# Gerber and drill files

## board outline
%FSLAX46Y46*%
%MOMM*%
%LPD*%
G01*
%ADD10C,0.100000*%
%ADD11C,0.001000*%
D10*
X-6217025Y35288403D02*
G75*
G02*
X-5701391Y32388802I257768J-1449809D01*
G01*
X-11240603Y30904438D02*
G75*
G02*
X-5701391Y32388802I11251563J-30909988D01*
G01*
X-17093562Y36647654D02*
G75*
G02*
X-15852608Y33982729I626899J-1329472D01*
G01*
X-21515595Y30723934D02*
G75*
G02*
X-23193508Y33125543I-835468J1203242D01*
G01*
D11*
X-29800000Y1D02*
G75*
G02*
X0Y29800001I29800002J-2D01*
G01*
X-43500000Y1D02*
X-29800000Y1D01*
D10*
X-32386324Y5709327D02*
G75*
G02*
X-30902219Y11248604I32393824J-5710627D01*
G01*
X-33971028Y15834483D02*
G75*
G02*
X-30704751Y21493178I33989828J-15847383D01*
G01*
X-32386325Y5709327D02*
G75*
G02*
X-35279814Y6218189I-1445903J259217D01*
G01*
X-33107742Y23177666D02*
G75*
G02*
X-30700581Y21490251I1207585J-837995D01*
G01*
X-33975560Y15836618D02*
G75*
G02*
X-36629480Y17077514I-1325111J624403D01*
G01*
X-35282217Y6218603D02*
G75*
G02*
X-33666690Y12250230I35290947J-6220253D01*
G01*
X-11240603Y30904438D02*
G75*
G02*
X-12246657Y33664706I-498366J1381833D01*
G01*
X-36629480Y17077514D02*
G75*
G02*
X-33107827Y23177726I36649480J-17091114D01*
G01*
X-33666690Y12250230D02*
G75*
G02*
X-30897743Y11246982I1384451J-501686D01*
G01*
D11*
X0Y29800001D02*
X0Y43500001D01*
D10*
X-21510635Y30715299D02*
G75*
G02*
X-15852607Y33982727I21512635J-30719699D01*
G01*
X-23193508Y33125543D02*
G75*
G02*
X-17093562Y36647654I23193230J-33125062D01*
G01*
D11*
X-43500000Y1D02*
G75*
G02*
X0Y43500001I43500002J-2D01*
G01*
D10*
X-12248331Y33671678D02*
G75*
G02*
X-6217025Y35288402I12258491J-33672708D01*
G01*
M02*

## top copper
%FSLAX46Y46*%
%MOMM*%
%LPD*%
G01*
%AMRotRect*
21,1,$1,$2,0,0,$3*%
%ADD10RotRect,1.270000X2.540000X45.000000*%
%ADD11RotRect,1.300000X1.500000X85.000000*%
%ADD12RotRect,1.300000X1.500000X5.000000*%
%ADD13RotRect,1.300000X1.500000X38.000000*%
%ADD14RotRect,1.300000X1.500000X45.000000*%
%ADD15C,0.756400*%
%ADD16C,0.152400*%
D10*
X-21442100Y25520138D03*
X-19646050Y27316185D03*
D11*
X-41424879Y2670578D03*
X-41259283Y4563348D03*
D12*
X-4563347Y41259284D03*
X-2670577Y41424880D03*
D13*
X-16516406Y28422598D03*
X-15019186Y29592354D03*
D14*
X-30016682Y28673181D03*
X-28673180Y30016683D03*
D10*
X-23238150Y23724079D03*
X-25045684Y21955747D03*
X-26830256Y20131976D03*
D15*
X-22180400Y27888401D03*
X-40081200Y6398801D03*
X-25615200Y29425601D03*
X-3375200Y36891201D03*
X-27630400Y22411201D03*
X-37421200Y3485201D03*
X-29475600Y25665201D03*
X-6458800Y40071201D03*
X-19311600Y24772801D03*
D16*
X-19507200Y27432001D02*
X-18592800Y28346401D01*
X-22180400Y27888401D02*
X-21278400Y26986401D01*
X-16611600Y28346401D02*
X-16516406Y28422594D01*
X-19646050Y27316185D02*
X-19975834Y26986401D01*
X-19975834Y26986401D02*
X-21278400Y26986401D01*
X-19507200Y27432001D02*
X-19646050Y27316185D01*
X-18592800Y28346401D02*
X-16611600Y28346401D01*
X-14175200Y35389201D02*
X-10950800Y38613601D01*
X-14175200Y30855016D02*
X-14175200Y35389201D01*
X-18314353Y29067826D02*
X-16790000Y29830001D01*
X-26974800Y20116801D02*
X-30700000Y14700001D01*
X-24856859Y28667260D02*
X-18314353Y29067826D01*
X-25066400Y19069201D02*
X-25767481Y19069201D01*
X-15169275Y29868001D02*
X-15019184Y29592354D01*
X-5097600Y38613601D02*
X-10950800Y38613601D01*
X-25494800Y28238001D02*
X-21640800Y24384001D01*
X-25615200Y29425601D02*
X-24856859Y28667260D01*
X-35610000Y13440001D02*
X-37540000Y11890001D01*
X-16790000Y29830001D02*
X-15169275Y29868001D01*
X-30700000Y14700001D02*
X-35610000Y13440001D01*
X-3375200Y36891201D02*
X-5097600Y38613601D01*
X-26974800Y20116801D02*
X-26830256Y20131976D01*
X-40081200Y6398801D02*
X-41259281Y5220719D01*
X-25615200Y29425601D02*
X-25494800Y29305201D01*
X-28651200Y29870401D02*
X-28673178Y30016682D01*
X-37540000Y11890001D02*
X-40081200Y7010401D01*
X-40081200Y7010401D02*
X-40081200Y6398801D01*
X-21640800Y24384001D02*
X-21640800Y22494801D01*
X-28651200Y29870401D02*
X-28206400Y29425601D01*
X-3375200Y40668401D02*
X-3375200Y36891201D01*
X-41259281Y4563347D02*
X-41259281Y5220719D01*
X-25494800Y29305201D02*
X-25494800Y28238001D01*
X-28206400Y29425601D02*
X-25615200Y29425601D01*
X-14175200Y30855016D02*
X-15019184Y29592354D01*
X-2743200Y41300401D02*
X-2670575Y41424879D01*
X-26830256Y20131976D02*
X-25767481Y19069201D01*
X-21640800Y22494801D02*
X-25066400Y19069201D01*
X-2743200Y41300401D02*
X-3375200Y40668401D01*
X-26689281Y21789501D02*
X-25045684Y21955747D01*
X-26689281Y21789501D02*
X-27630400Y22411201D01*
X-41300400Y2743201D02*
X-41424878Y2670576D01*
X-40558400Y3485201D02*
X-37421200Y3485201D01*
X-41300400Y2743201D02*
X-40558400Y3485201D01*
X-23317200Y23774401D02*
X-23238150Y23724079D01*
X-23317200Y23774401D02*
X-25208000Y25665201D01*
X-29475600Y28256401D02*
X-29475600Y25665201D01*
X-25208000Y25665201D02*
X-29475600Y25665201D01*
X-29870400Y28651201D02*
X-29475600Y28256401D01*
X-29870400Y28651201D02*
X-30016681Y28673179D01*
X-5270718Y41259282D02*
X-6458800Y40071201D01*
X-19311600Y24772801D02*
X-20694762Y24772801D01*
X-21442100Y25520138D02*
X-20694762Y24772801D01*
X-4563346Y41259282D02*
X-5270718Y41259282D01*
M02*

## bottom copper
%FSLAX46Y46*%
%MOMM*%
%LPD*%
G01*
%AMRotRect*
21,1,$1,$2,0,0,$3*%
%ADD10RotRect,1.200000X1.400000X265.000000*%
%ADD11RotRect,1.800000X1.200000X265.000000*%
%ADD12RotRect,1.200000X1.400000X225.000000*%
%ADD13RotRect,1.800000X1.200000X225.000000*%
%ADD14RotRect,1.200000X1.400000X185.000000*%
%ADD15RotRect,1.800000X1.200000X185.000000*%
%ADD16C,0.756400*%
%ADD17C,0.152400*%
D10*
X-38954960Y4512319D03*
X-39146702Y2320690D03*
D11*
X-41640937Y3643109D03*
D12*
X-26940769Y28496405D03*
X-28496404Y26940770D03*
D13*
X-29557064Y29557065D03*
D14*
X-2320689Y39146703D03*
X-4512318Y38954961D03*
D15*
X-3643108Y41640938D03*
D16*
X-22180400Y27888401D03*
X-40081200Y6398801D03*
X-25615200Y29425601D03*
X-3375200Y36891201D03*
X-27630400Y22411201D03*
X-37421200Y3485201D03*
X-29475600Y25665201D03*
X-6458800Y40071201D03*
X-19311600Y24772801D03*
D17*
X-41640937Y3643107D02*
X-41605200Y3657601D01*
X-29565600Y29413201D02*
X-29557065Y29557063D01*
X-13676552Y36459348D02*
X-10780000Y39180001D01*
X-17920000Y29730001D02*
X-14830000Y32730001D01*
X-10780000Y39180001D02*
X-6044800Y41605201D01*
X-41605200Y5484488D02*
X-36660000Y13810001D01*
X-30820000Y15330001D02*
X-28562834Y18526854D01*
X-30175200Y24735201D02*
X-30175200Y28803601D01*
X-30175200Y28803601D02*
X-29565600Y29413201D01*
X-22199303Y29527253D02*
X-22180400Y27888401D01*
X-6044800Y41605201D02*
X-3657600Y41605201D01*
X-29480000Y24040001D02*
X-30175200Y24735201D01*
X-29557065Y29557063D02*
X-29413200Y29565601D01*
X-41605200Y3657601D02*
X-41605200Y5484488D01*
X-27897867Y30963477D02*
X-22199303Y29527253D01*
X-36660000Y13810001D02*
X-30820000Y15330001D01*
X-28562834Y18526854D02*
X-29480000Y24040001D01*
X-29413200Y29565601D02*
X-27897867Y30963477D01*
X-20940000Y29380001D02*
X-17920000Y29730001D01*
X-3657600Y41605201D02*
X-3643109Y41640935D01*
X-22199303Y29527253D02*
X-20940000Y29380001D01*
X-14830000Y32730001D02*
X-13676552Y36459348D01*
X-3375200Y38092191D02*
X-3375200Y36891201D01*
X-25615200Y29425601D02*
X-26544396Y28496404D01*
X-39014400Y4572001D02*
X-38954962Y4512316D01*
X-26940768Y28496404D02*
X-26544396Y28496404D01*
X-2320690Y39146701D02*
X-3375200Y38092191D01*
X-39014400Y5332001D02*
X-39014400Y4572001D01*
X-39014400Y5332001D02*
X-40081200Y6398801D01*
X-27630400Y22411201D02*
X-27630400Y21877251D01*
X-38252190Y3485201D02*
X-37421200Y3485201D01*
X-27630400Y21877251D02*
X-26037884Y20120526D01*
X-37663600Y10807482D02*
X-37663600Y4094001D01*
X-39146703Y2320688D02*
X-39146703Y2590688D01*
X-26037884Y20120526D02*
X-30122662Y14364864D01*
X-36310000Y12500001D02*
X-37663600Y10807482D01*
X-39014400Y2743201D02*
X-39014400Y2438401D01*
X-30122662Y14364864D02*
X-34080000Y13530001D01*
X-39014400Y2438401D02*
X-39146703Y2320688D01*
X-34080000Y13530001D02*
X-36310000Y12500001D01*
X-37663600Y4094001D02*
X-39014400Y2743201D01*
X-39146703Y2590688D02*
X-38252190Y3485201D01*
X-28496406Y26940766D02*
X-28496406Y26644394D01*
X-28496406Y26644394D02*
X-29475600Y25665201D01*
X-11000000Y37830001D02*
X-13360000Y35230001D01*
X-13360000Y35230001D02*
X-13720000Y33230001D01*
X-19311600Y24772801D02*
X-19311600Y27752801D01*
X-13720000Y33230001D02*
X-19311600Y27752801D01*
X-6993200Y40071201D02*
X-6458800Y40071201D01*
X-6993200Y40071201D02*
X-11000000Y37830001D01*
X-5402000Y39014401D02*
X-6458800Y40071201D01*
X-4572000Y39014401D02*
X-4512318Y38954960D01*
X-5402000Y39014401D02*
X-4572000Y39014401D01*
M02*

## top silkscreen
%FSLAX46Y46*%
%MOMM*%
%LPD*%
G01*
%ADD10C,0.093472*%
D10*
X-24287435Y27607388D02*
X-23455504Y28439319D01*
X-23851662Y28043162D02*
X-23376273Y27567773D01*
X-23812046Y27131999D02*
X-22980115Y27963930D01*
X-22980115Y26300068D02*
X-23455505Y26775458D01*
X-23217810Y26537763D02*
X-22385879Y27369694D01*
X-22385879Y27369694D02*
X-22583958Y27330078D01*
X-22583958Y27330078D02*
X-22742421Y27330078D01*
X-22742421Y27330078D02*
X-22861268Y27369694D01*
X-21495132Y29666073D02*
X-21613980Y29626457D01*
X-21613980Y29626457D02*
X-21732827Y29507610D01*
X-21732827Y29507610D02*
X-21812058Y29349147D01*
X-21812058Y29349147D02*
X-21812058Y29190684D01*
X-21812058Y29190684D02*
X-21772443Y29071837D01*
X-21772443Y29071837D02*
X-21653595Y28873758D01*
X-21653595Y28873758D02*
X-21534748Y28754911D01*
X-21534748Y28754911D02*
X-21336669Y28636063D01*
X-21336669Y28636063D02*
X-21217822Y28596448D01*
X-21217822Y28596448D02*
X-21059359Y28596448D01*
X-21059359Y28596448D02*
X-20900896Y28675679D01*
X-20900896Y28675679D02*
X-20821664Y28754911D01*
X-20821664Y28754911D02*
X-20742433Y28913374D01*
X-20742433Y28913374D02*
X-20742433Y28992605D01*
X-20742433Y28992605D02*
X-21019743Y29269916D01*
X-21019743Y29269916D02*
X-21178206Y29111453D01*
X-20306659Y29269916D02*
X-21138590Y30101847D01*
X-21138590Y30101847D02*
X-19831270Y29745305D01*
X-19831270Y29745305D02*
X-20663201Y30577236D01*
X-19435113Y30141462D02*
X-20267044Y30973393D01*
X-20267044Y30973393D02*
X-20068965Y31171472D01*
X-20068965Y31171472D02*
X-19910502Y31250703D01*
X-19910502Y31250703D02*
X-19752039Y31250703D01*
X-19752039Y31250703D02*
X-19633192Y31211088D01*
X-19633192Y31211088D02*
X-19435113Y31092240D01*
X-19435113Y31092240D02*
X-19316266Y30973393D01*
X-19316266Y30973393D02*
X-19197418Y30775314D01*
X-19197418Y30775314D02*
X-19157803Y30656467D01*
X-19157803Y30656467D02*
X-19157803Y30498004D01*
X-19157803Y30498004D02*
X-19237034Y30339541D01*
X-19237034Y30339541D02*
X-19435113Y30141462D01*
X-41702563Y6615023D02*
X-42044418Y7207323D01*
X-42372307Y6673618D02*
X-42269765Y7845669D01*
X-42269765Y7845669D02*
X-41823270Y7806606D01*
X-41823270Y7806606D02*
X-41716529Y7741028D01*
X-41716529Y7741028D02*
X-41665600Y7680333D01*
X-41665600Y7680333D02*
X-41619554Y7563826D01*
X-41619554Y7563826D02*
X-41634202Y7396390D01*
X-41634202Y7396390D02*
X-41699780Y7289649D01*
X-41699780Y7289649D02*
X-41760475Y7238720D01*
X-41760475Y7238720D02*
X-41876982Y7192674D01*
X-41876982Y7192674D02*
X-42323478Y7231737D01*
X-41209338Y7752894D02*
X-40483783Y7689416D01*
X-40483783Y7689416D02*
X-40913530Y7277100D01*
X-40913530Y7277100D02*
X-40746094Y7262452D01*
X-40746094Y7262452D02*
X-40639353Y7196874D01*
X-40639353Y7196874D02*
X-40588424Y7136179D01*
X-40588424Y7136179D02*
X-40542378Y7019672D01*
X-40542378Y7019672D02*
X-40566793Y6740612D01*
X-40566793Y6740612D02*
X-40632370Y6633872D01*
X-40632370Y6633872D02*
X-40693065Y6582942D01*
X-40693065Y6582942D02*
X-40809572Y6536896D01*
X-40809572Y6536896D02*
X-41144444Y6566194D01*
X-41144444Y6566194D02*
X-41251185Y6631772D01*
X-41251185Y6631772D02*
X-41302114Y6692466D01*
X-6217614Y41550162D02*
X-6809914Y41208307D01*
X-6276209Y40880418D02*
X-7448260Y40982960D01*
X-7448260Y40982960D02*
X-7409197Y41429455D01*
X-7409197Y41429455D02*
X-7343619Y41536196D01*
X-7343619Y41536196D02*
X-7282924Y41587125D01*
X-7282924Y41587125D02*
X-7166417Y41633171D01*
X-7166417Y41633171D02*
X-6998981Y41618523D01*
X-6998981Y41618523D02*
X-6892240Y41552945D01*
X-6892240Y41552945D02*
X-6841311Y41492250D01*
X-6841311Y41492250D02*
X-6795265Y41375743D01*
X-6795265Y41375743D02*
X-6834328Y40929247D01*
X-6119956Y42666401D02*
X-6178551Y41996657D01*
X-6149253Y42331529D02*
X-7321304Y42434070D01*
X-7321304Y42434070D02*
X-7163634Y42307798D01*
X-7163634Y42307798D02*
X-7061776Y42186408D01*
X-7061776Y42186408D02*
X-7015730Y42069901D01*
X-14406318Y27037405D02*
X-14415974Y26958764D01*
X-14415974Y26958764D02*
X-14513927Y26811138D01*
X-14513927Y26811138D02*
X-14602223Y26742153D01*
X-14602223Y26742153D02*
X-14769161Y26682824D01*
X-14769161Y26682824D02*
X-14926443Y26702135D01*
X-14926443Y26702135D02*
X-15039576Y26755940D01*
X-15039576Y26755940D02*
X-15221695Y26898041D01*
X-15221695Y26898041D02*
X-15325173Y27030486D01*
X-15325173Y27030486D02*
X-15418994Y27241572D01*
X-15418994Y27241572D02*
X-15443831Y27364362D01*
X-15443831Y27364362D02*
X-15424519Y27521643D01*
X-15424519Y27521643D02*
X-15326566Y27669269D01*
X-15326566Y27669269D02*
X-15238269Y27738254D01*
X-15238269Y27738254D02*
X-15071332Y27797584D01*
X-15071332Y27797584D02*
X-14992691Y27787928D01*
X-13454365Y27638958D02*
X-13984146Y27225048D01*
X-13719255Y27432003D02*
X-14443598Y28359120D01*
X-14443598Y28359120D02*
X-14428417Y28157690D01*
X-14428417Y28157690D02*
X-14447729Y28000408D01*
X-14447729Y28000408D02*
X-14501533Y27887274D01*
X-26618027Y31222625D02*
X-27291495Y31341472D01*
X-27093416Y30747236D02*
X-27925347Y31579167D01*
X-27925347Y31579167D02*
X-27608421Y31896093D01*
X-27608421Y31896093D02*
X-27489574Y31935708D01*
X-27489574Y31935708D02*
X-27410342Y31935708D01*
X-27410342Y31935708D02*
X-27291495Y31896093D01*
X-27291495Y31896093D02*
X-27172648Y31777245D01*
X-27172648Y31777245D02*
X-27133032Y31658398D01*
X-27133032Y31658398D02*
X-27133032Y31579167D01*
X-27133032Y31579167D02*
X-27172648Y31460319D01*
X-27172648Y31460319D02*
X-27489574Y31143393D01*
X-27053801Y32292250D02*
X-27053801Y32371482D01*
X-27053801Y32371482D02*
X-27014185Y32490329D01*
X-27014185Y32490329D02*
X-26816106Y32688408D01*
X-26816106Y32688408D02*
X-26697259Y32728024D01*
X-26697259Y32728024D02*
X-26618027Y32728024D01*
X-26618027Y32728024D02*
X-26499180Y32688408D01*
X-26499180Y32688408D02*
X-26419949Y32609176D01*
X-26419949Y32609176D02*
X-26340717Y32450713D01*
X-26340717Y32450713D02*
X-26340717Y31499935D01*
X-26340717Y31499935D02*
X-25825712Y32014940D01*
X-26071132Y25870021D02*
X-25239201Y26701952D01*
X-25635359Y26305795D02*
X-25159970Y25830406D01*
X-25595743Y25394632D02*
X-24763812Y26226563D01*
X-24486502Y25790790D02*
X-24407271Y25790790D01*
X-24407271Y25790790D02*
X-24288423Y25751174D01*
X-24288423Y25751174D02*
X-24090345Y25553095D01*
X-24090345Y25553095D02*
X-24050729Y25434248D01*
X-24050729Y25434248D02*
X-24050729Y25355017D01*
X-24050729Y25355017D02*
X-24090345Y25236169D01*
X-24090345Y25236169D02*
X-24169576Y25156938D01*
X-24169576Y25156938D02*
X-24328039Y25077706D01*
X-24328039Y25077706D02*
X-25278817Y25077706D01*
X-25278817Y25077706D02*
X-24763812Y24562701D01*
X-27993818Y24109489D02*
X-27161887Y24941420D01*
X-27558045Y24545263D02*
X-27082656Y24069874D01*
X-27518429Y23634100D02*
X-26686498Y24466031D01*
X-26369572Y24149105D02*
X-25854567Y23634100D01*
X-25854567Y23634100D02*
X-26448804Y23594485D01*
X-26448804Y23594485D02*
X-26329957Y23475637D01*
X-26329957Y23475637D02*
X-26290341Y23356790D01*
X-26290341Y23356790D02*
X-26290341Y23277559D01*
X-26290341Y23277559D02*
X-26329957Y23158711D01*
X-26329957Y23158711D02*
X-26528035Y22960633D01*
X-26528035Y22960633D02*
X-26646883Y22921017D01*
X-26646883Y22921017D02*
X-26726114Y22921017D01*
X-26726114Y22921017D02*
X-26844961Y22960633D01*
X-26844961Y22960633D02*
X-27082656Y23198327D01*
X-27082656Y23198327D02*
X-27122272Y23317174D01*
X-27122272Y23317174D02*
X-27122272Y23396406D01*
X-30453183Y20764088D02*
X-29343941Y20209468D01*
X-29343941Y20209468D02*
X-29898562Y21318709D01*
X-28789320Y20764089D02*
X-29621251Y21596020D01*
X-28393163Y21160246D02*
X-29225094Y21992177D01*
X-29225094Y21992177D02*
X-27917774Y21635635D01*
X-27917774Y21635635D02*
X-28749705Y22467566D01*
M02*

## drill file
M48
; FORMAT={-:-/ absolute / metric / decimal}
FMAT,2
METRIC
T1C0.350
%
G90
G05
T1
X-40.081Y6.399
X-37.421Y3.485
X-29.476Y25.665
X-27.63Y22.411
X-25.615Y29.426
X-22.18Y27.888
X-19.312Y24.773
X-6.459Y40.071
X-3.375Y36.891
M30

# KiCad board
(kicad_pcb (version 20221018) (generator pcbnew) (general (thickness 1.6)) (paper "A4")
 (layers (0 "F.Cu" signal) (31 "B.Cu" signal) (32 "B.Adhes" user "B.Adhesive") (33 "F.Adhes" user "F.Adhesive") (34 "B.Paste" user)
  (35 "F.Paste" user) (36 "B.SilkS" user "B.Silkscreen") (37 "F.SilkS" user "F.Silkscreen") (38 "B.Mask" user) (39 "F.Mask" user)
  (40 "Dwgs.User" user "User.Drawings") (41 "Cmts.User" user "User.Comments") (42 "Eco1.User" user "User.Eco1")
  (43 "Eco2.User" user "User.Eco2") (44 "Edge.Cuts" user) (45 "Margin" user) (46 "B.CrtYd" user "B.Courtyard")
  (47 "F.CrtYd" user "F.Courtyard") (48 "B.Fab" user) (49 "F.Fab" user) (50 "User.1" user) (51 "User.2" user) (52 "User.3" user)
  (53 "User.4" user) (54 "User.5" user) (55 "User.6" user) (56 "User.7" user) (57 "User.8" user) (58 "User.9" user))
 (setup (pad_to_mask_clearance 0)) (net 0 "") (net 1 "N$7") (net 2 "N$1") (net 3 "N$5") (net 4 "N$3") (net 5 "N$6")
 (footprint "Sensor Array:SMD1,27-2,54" (layer "F.Cu") (at -21.4421 -25.520138 45)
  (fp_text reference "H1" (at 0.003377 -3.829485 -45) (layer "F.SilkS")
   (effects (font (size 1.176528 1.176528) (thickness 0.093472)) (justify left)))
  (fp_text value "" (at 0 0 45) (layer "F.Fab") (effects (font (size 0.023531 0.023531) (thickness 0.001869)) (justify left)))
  (pad "1" smd rect (at 0 0 45) (size 1.27 2.54) (layers "F.Cu" "F.Paste" "F.Mask") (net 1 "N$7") (solder_mask_margin 0.1016)
   (thermal_bridge_angle 45)))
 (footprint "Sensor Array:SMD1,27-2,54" (layer "F.Cu") (at -19.64605 -27.316185 45)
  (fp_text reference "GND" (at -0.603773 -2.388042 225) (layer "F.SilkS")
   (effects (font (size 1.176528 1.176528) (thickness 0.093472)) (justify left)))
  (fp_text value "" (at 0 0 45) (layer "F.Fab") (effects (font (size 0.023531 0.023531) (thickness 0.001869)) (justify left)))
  (pad "1" smd rect (at 0 0 45) (size 1.27 2.54) (layers "F.Cu" "F.Paste" "F.Mask") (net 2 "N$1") (solder_mask_margin 0.1016)
   (thermal_bridge_angle 45)))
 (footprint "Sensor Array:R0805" (layer "F.Cu") (at -41.342081 -3.616963 85)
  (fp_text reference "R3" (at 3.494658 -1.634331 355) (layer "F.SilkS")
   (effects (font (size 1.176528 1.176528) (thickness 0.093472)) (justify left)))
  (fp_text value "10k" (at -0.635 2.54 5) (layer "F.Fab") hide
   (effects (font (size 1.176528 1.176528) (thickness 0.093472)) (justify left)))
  (pad "1" smd rect (at -0.95 0 85) (size 1.3 1.5) (layers "F.Cu" "F.Paste" "F.Mask") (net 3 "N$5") (solder_mask_margin 0.1016)
   (thermal_bridge_angle 45))
  (pad "2" smd rect (at 0.95 0 85) (size 1.3 1.5) (layers "F.Cu" "F.Paste" "F.Mask") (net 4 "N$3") (solder_mask_margin 0.1016)
   (thermal_bridge_angle 45)))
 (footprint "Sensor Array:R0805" (layer "F.Cu") (at -3.616962 -41.342082 5)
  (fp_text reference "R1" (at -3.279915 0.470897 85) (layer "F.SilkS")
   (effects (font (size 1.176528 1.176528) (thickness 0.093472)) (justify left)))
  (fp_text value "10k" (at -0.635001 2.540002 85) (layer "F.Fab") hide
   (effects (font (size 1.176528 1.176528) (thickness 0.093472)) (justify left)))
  (pad "1" smd rect (at -0.95 0 5) (size 1.3 1.5) (layers "F.Cu" "F.Paste" "F.Mask") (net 1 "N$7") (solder_mask_margin 0.1016)
   (thermal_bridge_angle 45))
  (pad "2" smd rect (at 0.95 0 5) (size 1.3 1.5) (layers "F.Cu" "F.Paste" "F.Mask") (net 4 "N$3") (solder_mask_margin 0.1016)
   (thermal_bridge_angle 45)))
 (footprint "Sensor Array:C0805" (layer "F.Cu") (at -15.767796 -29.007476 38)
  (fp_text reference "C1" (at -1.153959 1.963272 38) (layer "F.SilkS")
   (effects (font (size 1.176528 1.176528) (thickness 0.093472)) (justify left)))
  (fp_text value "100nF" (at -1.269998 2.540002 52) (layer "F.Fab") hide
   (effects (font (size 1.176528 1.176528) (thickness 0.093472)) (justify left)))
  (pad "1" smd rect (at -0.95 0 38) (size 1.3 1.5) (layers "F.Cu" "F.Paste" "F.Mask") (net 2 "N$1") (solder_mask_margin 0.1016)
   (thermal_bridge_angle 45))
  (pad "2" smd rect (at 0.95 0 38) (size 1.3 1.5) (layers "F.Cu" "F.Paste" "F.Mask") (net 4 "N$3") (solder_mask_margin 0.1016)
   (thermal_bridge_angle 45)))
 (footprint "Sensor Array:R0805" (layer "F.Cu") (at -29.344931 -29.344932 45)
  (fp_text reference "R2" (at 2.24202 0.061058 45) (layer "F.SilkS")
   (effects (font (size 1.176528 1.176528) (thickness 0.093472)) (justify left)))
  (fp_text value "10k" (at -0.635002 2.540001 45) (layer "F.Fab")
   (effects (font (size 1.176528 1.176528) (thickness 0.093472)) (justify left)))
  (pad "1" smd rect (at -0.95 0 45) (size 1.3 1.5) (layers "F.Cu" "F.Paste" "F.Mask") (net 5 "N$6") (solder_mask_margin 0.1016)
   (thermal_bridge_angle 45))
  (pad "2" smd rect (at 0.95 0 45) (size 1.3 1.5) (layers "F.Cu" "F.Paste" "F.Mask") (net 4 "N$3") (solder_mask_margin 0.1016)
   (thermal_bridge_angle 45)))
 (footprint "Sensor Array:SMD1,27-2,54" (layer "F.Cu") (at -23.23815 -23.724079 45)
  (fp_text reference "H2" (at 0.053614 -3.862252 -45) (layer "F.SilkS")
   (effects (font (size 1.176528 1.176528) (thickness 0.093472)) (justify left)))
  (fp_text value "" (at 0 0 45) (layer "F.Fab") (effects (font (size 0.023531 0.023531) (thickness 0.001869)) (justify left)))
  (pad "1" smd rect (at 0 0 45) (size 1.27 2.54) (layers "F.Cu" "F.Paste" "F.Mask") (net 5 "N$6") (solder_mask_margin 0.1016)
   (thermal_bridge_angle 45)))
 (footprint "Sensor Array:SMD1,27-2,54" (layer "F.Cu") (at -25.045684 -21.955747 45)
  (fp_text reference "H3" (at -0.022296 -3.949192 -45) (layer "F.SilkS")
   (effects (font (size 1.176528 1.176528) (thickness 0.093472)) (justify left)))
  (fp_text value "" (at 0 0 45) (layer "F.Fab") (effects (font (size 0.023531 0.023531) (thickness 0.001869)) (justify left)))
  (pad "1" smd rect (at 0 0 45) (size 1.27 2.54) (layers "F.Cu" "F.Paste" "F.Mask") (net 3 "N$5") (solder_mask_margin 0.1016)
   (thermal_bridge_angle 45)))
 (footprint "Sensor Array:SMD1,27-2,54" (layer "F.Cu") (at -26.830256 -20.131976 45)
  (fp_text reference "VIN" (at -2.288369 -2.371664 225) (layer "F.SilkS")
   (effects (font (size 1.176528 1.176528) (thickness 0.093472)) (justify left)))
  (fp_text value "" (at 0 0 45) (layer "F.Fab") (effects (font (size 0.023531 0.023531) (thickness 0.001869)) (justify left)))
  (pad "1" smd rect (at 0 0 45) (size 1.27 2.54) (layers "F.Cu" "F.Paste" "F.Mask") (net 4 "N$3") (solder_mask_margin 0.1016)
   (thermal_bridge_angle 45)))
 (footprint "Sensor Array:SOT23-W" (layer "B.Cu") (at -40.345884 -3.529807 -95)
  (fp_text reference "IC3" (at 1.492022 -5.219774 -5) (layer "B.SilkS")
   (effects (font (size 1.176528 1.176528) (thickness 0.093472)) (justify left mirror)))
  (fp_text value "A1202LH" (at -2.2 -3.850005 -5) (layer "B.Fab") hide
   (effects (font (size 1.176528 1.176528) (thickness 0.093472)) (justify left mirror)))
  (pad "1" smd rect (at -1.1 -1.3 265) (size 1.2 1.4) (layers "B.Cu" "B.Paste" "B.Mask") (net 4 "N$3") (solder_mask_margin 0.1016)
   (thermal_bridge_angle 45))
  (pad "2" smd rect (at 1.1 -1.3 265) (size 1.2 1.4) (layers "B.Cu" "B.Paste" "B.Mask") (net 3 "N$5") (solder_mask_margin 0.1016)
   (thermal_bridge_angle 45))
  (pad "3" smd rect (at 0 1.3 265) (size 1.8 1.2) (layers "B.Cu" "B.Paste" "B.Mask") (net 2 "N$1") (solder_mask_margin 0.1016)
   (thermal_bridge_angle 45)))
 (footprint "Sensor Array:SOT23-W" (layer "B.Cu") (at -28.637825 -28.637826 -135)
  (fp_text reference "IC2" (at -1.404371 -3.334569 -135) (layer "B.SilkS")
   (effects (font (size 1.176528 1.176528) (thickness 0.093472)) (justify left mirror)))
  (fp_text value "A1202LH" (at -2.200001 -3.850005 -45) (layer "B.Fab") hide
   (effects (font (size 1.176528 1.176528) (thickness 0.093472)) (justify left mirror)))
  (pad "1" smd rect (at -1.1 -1.3 225) (size 1.2 1.4) (layers "B.Cu" "B.Paste" "B.Mask") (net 4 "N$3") (solder_mask_margin 0.1016)
   (thermal_bridge_angle 45))
  (pad "2" smd rect (at 1.1 -1.3 225) (size 1.2 1.4) (layers "B.Cu" "B.Paste" "B.Mask") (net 5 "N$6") (solder_mask_margin 0.1016)
   (thermal_bridge_angle 45))
  (pad "3" smd rect (at 0 1.3 225) (size 1.8 1.2) (layers "B.Cu" "B.Paste" "B.Mask") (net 2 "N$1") (solder_mask_margin 0.1016)
   (thermal_bridge_angle 45)))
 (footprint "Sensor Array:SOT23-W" (layer "B.Cu") (at -3.529806 -40.345885 -175)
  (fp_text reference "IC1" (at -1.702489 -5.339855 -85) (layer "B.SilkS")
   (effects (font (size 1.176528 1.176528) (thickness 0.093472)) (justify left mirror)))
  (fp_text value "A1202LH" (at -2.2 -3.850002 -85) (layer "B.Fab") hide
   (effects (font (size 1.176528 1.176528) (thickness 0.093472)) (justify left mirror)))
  (pad "1" smd rect (at -1.1 -1.3 185) (size 1.2 1.4) (layers "B.Cu" "B.Paste" "B.Mask") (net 4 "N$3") (solder_mask_margin 0.1016)
   (thermal_bridge_angle 45))
  (pad "2" smd rect (at 1.1 -1.3 185) (size 1.2 1.4) (layers "B.Cu" "B.Paste" "B.Mask") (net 1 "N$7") (solder_mask_margin 0.1016)
   (thermal_bridge_angle 45))
  (pad "3" smd rect (at 0 1.3 185) (size 1.8 1.2) (layers "B.Cu" "B.Paste" "B.Mask") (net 2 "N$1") (solder_mask_margin 0.1016)
   (thermal_bridge_angle 45)))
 (gr_arc (start -6.217025 -35.288403) (mid -4.509456 -34.096408) (end -5.701391 -32.388802) (stroke (width 0.1) (type default))
  (layer "Edge.Cuts"))
 (gr_arc (start -11.240603 -30.904438) (mid -8.503406 -31.767561) (end -5.701391 -32.388802) (stroke (width 0.1) (type default))
  (layer "Edge.Cuts"))
 (gr_arc (start -17.093562 -36.647654) (mid -15.134188 -35.938672) (end -15.852608 -33.98273) (stroke (width 0.1) (type default))
  (layer "Edge.Cuts"))
 (gr_arc (start -21.515595 -30.723934) (mid -23.551878 -31.088224) (end -23.193508 -33.125543) (stroke (width 0.1) (type default))
  (layer "Edge.Cuts"))
 (gr_arc (start -29.8 -0.000001) (mid -21.071782 -21.071782) (end 0 -29.800001) (stroke (width 0.001) (type solid)) (layer "Edge.Cuts"))
 (gr_line (start -43.5 -0.000001) (end -29.8 -0.000001) (stroke (width 0.001) (type solid)) (layer "Edge.Cuts"))
 (gr_arc (start -32.386324 -5.709327) (mid -31.765216 -8.511369) (end -30.902217 -11.248603) (stroke (width 0.1) (type default))
  (layer "Edge.Cuts"))
 (gr_arc (start -33.971028 -15.834483) (mid -32.461355 -18.735096) (end -30.704748 -21.493176) (stroke (width 0.1) (type default))
  (layer "Edge.Cuts"))
 (gr_arc (start -32.386325 -5.709327) (mid -34.086699 -4.521798) (end -35.279814 -6.218189) (stroke (width 0.1) (type default))
  (layer "Edge.Cuts"))
 (gr_arc (start -33.107742 -23.177666) (mid -31.056451 -23.543273) (end -30.700581 -21.490251) (stroke (width 0.1) (type default))
  (layer "Edge.Cuts"))
 (gr_arc (start -33.97556 -15.836618) (mid -35.921101 -15.134045) (end -36.62948 -17.077514) (stroke (width 0.1) (type default))
  (layer "Edge.Cuts"))
 (gr_arc (start -35.282217 -6.218603) (mid -34.60608 -9.269672) (end -33.66669 -12.25023) (stroke (width 0.1) (type default))
  (layer "Edge.Cuts"))
 (gr_arc (start -11.240603 -30.904438) (mid -13.119116 -31.783255) (end -12.246657 -33.664706) (stroke (width 0.1) (type default))
  (layer "Edge.Cuts"))
 (gr_arc (start -36.62948 -17.077514) (mid -35.001726 -20.204443) (end -33.107827 -23.177726) (stroke (width 0.1) (type default))
  (layer "Edge.Cuts"))
 (gr_arc (start -33.66669 -12.25023) (mid -31.780648 -13.13303) (end -30.897742 -11.246982) (stroke (width 0.1) (type default))
  (layer "Edge.Cuts"))
 (gr_line (start 0 -29.800001) (end 0 -43.500001) (stroke (width 0.001) (type solid)) (layer "Edge.Cuts"))
 (gr_arc (start -21.510635 -30.715299) (mid -18.752912 -32.472465) (end -15.852608 -33.98273) (stroke (width 0.1) (type default))
  (layer "Edge.Cuts"))
 (gr_arc (start -23.193508 -33.125543) (mid -20.22037 -35.019669) (end -17.093562 -36.647654) (stroke (width 0.1) (type default))
  (layer "Edge.Cuts"))
 (gr_arc (start -43.5 -0.000001) (mid -30.759145 -30.759145) (end 0 -43.500001) (stroke (width 0.001) (type solid)) (layer "Edge.Cuts"))
 (gr_arc (start -12.248331 -33.671678) (mid -9.26796 -34.611661) (end -6.217025 -35.288403) (stroke (width 0.1) (type default))
  (layer "Edge.Cuts"))
 (segment (start -19.5072 -27.432001) (end -18.5928 -28.346401) (width 0.1524) (layer "F.Cu") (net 2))
 (segment (start -22.1804 -27.888401) (end -21.2784 -26.986401) (width 0.1524) (layer "F.Cu") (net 2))
 (segment (start -16.6116 -28.346401) (end -16.516406 -28.422594) (width 0.1524) (layer "F.Cu") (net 2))
 (segment (start -19.64605 -27.316185) (end -19.975834 -26.986401) (width 0.1524) (layer "F.Cu") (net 2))
 (segment (start -19.975834 -26.986401) (end -21.2784 -26.986401) (width 0.1524) (layer "F.Cu") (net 2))
 (segment (start -19.5072 -27.432001) (end -19.64605 -27.316185) (width 0.1524) (layer "F.Cu") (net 2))
 (segment (start -18.5928 -28.346401) (end -16.6116 -28.346401) (width 0.1524) (layer "F.Cu") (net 2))
 (via (at -22.1804 -27.888401) (size 0.7564) (drill 0.35) (layers "F.Cu" "B.Cu") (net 2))
 (segment (start -41.640937 -3.643107) (end -41.6052 -3.657601) (width 0.1524) (layer "B.Cu") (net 2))
 (segment (start -29.5656 -29.413201) (end -29.557065 -29.557063) (width 0.1524) (layer "B.Cu") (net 2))
 (segment (start -13.676552 -36.459348) (end -10.78 -39.180001) (width 0.1524) (layer "B.Cu") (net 2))
 (segment (start -17.92 -29.730001) (end -14.83 -32.730001) (width 0.1524) (layer "B.Cu") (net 2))
 (segment (start -10.78 -39.180001) (end -6.0448 -41.605201) (width 0.1524) (layer "B.Cu") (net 2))
 (segment (start -41.6052 -5.484488) (end -36.66 -13.810001) (width 0.1524) (layer "B.Cu") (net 2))
 (segment (start -30.82 -15.330001) (end -28.562834 -18.526854) (width 0.1524) (layer "B.Cu") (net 2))
 (segment (start -30.1752 -24.735201) (end -30.1752 -28.803601) (width 0.1524) (layer "B.Cu") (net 2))
 (segment (start -30.1752 -28.803601) (end -29.5656 -29.413201) (width 0.1524) (layer "B.Cu") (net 2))
 (segment (start -22.199303 -29.527253) (end -22.1804 -27.888401) (width 0.1524) (layer "B.Cu") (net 2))
 (segment (start -6.0448 -41.605201) (end -3.6576 -41.605201) (width 0.1524) (layer "B.Cu") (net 2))
 (segment (start -29.48 -24.040001) (end -30.1752 -24.735201) (width 0.1524) (layer "B.Cu") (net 2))
 (segment (start -29.557065 -29.557063) (end -29.4132 -29.565601) (width 0.1524) (layer "B.Cu") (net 2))
 (segment (start -41.6052 -3.657601) (end -41.6052 -5.484488) (width 0.1524) (layer "B.Cu") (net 2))
 (segment (start -27.897867 -30.963477) (end -22.199303 -29.527253) (width 0.1524) (layer "B.Cu") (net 2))
 (segment (start -36.66 -13.810001) (end -30.82 -15.330001) (width 0.1524) (layer "B.Cu") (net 2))
 (segment (start -28.562834 -18.526854) (end -29.48 -24.040001) (width 0.1524) (layer "B.Cu") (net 2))
 (segment (start -29.4132 -29.565601) (end -27.897867 -30.963477) (width 0.1524) (layer "B.Cu") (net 2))
 (segment (start -20.94 -29.380001) (end -17.92 -29.730001) (width 0.1524) (layer "B.Cu") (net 2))
 (segment (start -3.6576 -41.605201) (end -3.643109 -41.640935) (width 0.1524) (layer "B.Cu") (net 2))
 (segment (start -22.199303 -29.527253) (end -20.94 -29.380001) (width 0.1524) (layer "B.Cu") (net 2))
 (segment (start -14.83 -32.730001) (end -13.676552 -36.459348) (width 0.1524) (layer "B.Cu") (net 2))
 (segment (start -14.1752 -35.389201) (end -10.9508 -38.613601) (width 0.1524) (layer "F.Cu") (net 4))
 (segment (start -14.1752 -30.855016) (end -14.1752 -35.389201) (width 0.1524) (layer "F.Cu") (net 4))
 (segment (start -18.314353 -29.067826) (end -16.79 -29.830001) (width 0.1524) (layer "F.Cu") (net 4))
 (segment (start -26.9748 -20.116801) (end -30.7 -14.700001) (width 0.1524) (layer "F.Cu") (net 4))
 (segment (start -24.856859 -28.66726) (end -18.314353 -29.067826) (width 0.1524) (layer "F.Cu") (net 4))
 (segment (start -25.0664 -19.069201) (end -25.767481 -19.069201) (width 0.1524) (layer "F.Cu") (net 4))
 (segment (start -15.169275 -29.868001) (end -15.019184 -29.592354) (width 0.1524) (layer "F.Cu") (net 4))
 (segment (start -5.0976 -38.613601) (end -10.9508 -38.613601) (width 0.1524) (layer "F.Cu") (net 4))
 (segment (start -25.4948 -28.238001) (end -21.6408 -24.384001) (width 0.1524) (layer "F.Cu") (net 4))
 (segment (start -25.6152 -29.425601) (end -24.856859 -28.66726) (width 0.1524) (layer "F.Cu") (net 4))
 (segment (start -35.61 -13.440001) (end -37.54 -11.890001) (width 0.1524) (layer "F.Cu") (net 4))
 (segment (start -16.79 -29.830001) (end -15.169275 -29.868001) (width 0.1524) (layer "F.Cu") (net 4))
 (segment (start -30.7 -14.700001) (end -35.61 -13.440001) (width 0.1524) (layer "F.Cu") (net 4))
 (segment (start -3.3752 -36.891201) (end -5.0976 -38.613601) (width 0.1524) (layer "F.Cu") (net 4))
 (segment (start -26.9748 -20.116801) (end -26.830256 -20.131976) (width 0.1524) (layer "F.Cu") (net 4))
 (segment (start -40.0812 -6.398801) (end -41.259281 -5.220719) (width 0.1524) (layer "F.Cu") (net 4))
 (segment (start -25.6152 -29.425601) (end -25.4948 -29.305201) (width 0.1524) (layer "F.Cu") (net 4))
 (segment (start -28.6512 -29.870401) (end -28.673178 -30.016682) (width 0.1524) (layer "F.Cu") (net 4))
 (segment (start -37.54 -11.890001) (end -40.0812 -7.010401) (width 0.1524) (layer "F.Cu") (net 4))
 (segment (start -40.0812 -7.010401) (end -40.0812 -6.398801) (width 0.1524) (layer "F.Cu") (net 4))
 (segment (start -21.6408 -24.384001) (end -21.6408 -22.494801) (width 0.1524) (layer "F.Cu") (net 4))
 (segment (start -28.6512 -29.870401) (end -28.2064 -29.425601) (width 0.1524) (layer "F.Cu") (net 4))
 (segment (start -3.3752 -40.668401) (end -3.3752 -36.891201) (width 0.1524) (layer "F.Cu") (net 4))
 (segment (start -41.259281 -4.563347) (end -41.259281 -5.220719) (width 0.1524) (layer "F.Cu") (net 4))
 (segment (start -25.4948 -29.305201) (end -25.4948 -28.238001) (width 0.1524) (layer "F.Cu") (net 4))
 (segment (start -28.2064 -29.425601) (end -25.6152 -29.425601) (width 0.1524) (layer "F.Cu") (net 4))
 (segment (start -14.1752 -30.855016) (end -15.019184 -29.592354) (width 0.1524) (layer "F.Cu") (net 4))
 (segment (start -2.7432 -41.300401) (end -2.670575 -41.424879) (width 0.1524) (layer "F.Cu") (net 4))
 (segment (start -26.830256 -20.131976) (end -25.767481 -19.069201) (width 0.1524) (layer "F.Cu") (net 4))
 (segment (start -21.6408 -22.494801) (end -25.0664 -19.069201) (width 0.1524) (layer "F.Cu") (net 4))
 (segment (start -2.7432 -41.300401) (end -3.3752 -40.668401) (width 0.1524) (layer "F.Cu") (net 4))
 (via (at -40.0812 -6.398801) (size 0.7564) (drill 0.35) (layers "F.Cu" "B.Cu") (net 4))
 (via (at -25.6152 -29.425601) (size 0.7564) (drill 0.35) (layers "F.Cu" "B.Cu") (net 4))
 (via (at -3.3752 -36.891201) (size 0.7564) (drill 0.35) (layers "F.Cu" "B.Cu") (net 4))
 (segment (start -3.3752 -38.092191) (end -3.3752 -36.891201) (width 0.1524) (layer "B.Cu") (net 4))
 (segment (start -25.6152 -29.425601) (end -26.544396 -28.496404) (width 0.1524) (layer "B.Cu") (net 4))
 (segment (start -39.0144 -4.572001) (end -38.954962 -4.512316) (width 0.1524) (layer "B.Cu") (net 4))
 (segment (start -26.940768 -28.496404) (end -26.544396 -28.496404) (width 0.1524) (layer "B.Cu") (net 4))
 (segment (start -2.32069 -39.146701) (end -3.3752 -38.092191) (width 0.1524) (layer "B.Cu") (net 4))
 (segment (start -39.0144 -5.332001) (end -39.0144 -4.572001) (width 0.1524) (layer "B.Cu") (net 4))
 (segment (start -39.0144 -5.332001) (end -40.0812 -6.398801) (width 0.1524) (layer "B.Cu") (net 4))
 (segment (start -26.689281 -21.789501) (end -25.045684 -21.955747) (width 0.1524) (layer "F.Cu") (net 3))
 (segment (start -26.689281 -21.789501) (end -27.6304 -22.411201) (width 0.1524) (layer "F.Cu") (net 3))
 (segment (start -41.3004 -2.743201) (end -41.424878 -2.670576) (width 0.1524) (layer "F.Cu") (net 3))
 (segment (start -40.5584 -3.485201) (end -37.4212 -3.485201) (width 0.1524) (layer "F.Cu") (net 3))
 (segment (start -41.3004 -2.743201) (end -40.5584 -3.485201) (width 0.1524) (layer "F.Cu") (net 3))
 (via (at -27.6304 -22.411201) (size 0.7564) (drill 0.35) (layers "F.Cu" "B.Cu") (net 3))
 (via (at -37.4212 -3.485201) (size 0.7564) (drill 0.35) (layers "F.Cu" "B.Cu") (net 3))
 (segment (start -27.6304 -22.411201) (end -27.6304 -21.877251) (width 0.1524) (layer "B.Cu") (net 3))
 (segment (start -38.25219 -3.485201) (end -37.4212 -3.485201) (width 0.1524) (layer "B.Cu") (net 3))
 (segment (start -27.6304 -21.877251) (end -26.037884 -20.120526) (width 0.1524) (layer "B.Cu") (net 3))
 (segment (start -37.6636 -10.807482) (end -37.6636 -4.094001) (width 0.1524) (layer "B.Cu") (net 3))
 (segment (start -39.146703 -2.320688) (end -39.146703 -2.590688) (width 0.1524) (layer "B.Cu") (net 3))
 (segment (start -26.037884 -20.120526) (end -30.122662 -14.364864) (width 0.1524) (layer "B.Cu") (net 3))
 (segment (start -36.31 -12.500001) (end -37.6636 -10.807482) (width 0.1524) (layer "B.Cu") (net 3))
 (segment (start -39.0144 -2.743201) (end -39.0144 -2.438401) (width 0.1524) (layer "B.Cu") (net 3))
 (segment (start -30.122662 -14.364864) (end -34.08 -13.530001) (width 0.1524) (layer "B.Cu") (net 3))
 (segment (start -39.0144 -2.438401) (end -39.146703 -2.320688) (width 0.1524) (layer "B.Cu") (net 3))
 (segment (start -34.08 -13.530001) (end -36.31 -12.500001) (width 0.1524) (layer "B.Cu") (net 3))
 (segment (start -37.6636 -4.094001) (end -39.0144 -2.743201) (width 0.1524) (layer "B.Cu") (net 3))
 (segment (start -39.146703 -2.590688) (end -38.25219 -3.485201) (width 0.1524) (layer "B.Cu") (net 3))
 (segment (start -23.3172 -23.774401) (end -23.23815 -23.724079) (width 0.1524) (layer "F.Cu") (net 5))
 (segment (start -23.3172 -23.774401) (end -25.208 -25.665201) (width 0.1524) (layer "F.Cu") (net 5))
 (segment (start -29.4756 -28.256401) (end -29.4756 -25.665201) (width 0.1524) (layer "F.Cu") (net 5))
 (segment (start -25.208 -25.665201) (end -29.4756 -25.665201) (width 0.1524) (layer "F.Cu") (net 5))
 (segment (start -29.8704 -28.651201) (end -29.4756 -28.256401) (width 0.1524) (layer "F.Cu") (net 5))
 (segment (start -29.8704 -28.651201) (end -30.016681 -28.673179) (width 0.1524) (layer "F.Cu") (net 5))
 (via (at -29.4756 -25.665201) (size 0.7564) (drill 0.35) (layers "F.Cu" "B.Cu") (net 5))
 (segment (start -28.496406 -26.940766) (end -28.496406 -26.644394) (width 0.1524) (layer "B.Cu") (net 5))
 (segment (start -28.496406 -26.644394) (end -29.4756 -25.665201) (width 0.1524) (layer "B.Cu") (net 5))
 (segment (start -5.270718 -41.259282) (end -6.4588 -40.071201) (width 0.1524) (layer "F.Cu") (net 1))
 (segment (start -19.3116 -24.772801) (end -20.694762 -24.772801) (width 0.1524) (layer "F.Cu") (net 1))
 (segment (start -21.4421 -25.520138) (end -20.694762 -24.772801) (width 0.1524) (layer "F.Cu") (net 1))
 (segment (start -4.563346 -41.259282) (end -5.270718 -41.259282) (width 0.1524) (layer "F.Cu") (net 1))
 (via (at -6.4588 -40.071201) (size 0.7564) (drill 0.35) (layers "F.Cu" "B.Cu") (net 1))
 (via (at -19.3116 -24.772801) (size 0.7564) (drill 0.35) (layers "F.Cu" "B.Cu") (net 1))
 (segment (start -11 -37.830001) (end -13.36 -35.230001) (width 0.1524) (layer "B.Cu") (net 1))
 (segment (start -13.36 -35.230001) (end -13.72 -33.230001) (width 0.1524) (layer "B.Cu") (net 1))
 (segment (start -19.3116 -24.772801) (end -19.3116 -27.752801) (width 0.1524) (layer "B.Cu") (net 1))
 (segment (start -13.72 -33.230001) (end -19.3116 -27.752801) (width 0.1524) (layer "B.Cu") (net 1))
 (segment (start -6.9932 -40.071201) (end -6.4588 -40.071201) (width 0.1524) (layer "B.Cu") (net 1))
 (segment (start -6.9932 -40.071201) (end -11 -37.830001) (width 0.1524) (layer "B.Cu") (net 1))
 (segment (start -5.402 -39.014401) (end -6.4588 -40.071201) (width 0.1524) (layer "B.Cu") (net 1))
 (segment (start -4.572 -39.014401) (end -4.512318 -38.95496) (width 0.1524) (layer "B.Cu") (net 1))
 (segment (start -5.402 -39.014401) (end -4.572 -39.014401) (width 0.1524) (layer "B.Cu") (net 1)))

